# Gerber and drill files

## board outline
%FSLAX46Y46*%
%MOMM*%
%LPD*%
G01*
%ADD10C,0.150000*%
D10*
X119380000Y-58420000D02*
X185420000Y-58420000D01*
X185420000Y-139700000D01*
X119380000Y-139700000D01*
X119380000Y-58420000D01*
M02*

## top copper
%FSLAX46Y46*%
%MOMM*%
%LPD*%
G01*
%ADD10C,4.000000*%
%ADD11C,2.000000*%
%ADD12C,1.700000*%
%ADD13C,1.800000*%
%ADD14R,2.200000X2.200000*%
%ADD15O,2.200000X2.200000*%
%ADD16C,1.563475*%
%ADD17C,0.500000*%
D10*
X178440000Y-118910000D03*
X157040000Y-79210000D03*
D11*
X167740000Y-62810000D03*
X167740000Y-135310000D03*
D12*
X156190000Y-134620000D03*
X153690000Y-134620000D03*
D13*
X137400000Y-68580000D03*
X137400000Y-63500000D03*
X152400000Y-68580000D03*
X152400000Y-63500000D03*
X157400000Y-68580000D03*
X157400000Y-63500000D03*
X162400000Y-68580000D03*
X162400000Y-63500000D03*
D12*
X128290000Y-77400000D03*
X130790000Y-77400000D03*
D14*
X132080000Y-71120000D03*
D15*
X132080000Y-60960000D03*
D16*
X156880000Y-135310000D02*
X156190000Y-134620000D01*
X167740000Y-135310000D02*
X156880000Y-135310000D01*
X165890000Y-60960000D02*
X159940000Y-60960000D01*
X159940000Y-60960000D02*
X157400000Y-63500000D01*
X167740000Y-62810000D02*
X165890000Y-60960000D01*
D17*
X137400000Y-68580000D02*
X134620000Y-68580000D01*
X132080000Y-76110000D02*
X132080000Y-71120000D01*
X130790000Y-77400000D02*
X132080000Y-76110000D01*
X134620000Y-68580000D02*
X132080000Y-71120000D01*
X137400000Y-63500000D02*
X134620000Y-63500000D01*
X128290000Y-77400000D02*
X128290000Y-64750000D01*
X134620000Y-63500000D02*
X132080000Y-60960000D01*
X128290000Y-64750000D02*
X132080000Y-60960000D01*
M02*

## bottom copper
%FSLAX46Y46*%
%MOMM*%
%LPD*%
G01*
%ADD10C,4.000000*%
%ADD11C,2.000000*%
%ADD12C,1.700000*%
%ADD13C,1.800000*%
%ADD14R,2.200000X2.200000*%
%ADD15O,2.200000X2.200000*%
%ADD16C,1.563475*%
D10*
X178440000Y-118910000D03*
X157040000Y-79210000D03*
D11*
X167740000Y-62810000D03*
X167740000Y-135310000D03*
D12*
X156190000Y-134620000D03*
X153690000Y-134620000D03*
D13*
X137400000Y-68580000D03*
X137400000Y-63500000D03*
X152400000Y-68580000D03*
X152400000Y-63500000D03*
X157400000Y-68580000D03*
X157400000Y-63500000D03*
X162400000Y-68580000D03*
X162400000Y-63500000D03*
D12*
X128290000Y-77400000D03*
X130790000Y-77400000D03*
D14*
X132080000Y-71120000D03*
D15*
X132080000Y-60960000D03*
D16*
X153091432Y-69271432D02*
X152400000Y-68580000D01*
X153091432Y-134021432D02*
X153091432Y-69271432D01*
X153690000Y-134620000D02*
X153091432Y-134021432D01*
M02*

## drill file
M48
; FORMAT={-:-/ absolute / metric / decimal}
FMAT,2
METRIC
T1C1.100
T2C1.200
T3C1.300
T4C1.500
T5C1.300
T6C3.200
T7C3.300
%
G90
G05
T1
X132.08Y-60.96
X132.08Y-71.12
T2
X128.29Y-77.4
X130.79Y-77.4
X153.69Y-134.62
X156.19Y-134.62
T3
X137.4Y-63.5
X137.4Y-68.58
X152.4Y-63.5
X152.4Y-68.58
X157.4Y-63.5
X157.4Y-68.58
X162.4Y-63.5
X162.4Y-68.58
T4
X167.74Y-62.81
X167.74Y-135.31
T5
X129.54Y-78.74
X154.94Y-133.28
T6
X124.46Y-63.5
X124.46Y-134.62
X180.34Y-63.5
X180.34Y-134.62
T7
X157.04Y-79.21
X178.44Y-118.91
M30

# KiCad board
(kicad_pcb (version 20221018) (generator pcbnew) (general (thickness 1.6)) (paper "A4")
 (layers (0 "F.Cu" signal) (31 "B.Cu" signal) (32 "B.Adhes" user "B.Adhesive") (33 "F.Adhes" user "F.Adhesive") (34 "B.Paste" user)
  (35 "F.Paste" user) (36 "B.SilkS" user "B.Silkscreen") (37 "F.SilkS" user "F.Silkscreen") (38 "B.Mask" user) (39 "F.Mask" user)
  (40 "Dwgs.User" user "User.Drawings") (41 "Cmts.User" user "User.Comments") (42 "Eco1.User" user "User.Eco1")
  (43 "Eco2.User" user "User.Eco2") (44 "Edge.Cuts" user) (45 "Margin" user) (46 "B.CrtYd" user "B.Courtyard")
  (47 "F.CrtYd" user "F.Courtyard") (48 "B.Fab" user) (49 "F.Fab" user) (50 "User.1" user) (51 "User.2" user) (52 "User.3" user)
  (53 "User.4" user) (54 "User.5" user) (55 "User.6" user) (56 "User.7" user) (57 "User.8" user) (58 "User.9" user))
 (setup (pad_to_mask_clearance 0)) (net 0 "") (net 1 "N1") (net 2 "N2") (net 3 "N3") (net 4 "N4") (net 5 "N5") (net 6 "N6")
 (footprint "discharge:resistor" (layer "F.Cu") (at 152.74 124.56 90)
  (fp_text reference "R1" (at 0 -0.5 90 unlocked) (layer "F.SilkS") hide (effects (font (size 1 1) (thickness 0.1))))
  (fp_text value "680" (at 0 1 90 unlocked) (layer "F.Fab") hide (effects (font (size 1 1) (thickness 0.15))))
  (pad "" np_thru_hole circle (at 5.65 25.7 90) (size 4 4) (drill 3.3) (layers "F&B.Cu" "*.Mask"))
  (pad "" np_thru_hole circle (at 45.35 4.3 90) (size 4 4) (drill 3.3) (layers "F&B.Cu" "*.Mask"))
  (pad "1" thru_hole circle (at 61.75 15 90) (size 2 2) (drill 1.5) (layers "*.Cu" "*.Mask") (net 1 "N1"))
  (pad "2" thru_hole circle (at -10.75 15 90) (size 2 2) (drill 1.5) (layers "*.Cu" "*.Mask") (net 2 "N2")))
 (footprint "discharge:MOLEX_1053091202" (layer "F.Cu") (at 156.19 134.62 180)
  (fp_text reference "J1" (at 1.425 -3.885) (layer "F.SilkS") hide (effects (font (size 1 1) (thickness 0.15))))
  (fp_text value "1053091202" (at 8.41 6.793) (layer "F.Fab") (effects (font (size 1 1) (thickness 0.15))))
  (pad "" np_thru_hole circle (at 1.25 1.34 180) (size 1.3 1.3) (drill 1.3) (layers "*.Cu" "*.Mask"))
  (pad "1" thru_hole circle (at 0 0 180) (size 1.7 1.7) (drill 1.2) (layers "*.Cu") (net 2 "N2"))
  (pad "2" thru_hole circle (at 2.5 0 180) (size 1.7 1.7) (drill 1.2) (layers "*.Cu") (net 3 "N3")))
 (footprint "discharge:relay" (layer "F.Cu") (at 134.68 72.39 90)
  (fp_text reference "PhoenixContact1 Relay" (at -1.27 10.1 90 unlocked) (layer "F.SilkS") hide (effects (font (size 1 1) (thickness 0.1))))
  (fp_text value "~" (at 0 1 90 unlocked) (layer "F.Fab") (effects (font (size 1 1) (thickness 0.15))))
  (pad "1" thru_hole circle (at 3.81 2.72 90) (size 1.8 1.8) (drill 1.3) (layers "*.Cu" "*.Mask") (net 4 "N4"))
  (pad "2" thru_hole circle (at 8.89 2.72 90) (size 1.8 1.8) (drill 1.3) (layers "*.Cu" "*.Mask") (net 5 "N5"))
  (pad "3" thru_hole circle (at 3.81 17.72 90) (size 1.8 1.8) (drill 1.3) (layers "*.Cu" "*.Mask") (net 3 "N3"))
  (pad "3" thru_hole circle (at 8.89 17.72 90) (size 1.8 1.8) (drill 1.3) (layers "*.Cu" "*.Mask") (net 3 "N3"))
  (pad "4" thru_hole circle (at 3.81 22.72 90) (size 1.8 1.8) (drill 1.3) (layers "*.Cu" "*.Mask") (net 1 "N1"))
  (pad "4" thru_hole circle (at 8.89 22.72 90) (size 1.8 1.8) (drill 1.3) (layers "*.Cu" "*.Mask") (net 1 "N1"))
  (pad "5" thru_hole circle (at 3.81 27.72 90) (size 1.8 1.8) (drill 1.3) (layers "*.Cu" "*.Mask") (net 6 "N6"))
  (pad "5" thru_hole circle (at 8.89 27.72 90) (size 1.8 1.8) (drill 1.3) (layers "*.Cu" "*.Mask") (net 6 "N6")))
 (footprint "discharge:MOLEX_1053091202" (layer "F.Cu") (at 128.29 77.4)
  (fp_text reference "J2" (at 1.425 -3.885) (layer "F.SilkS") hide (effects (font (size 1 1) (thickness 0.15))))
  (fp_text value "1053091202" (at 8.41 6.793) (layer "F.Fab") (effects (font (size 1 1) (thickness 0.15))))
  (pad "" np_thru_hole circle (at 1.25 1.34) (size 1.3 1.3) (drill 1.3) (layers "*.Cu" "*.Mask"))
  (pad "1" thru_hole circle (at 0 0) (size 1.7 1.7) (drill 1.2) (layers "*.Cu") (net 5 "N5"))
  (pad "2" thru_hole circle (at 2.5 0) (size 1.7 1.7) (drill 1.2) (layers "*.Cu") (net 4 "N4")))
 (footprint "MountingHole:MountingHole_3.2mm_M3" (layer "F.Cu") (at 124.46 134.62)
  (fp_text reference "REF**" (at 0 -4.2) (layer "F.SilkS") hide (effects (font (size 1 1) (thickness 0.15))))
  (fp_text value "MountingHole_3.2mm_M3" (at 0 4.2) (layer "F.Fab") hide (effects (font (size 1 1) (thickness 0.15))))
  (pad "" np_thru_hole circle (at 0 0) (size 3.2 3.2) (drill 3.2) (layers "F&B.Cu" "*.Mask")))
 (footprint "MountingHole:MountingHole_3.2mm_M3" (layer "F.Cu") (at 124.46 63.5)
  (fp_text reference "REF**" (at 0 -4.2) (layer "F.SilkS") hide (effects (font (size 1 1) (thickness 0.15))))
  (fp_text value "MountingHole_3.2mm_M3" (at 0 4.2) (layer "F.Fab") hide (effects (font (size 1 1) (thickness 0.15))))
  (pad "" np_thru_hole circle (at 0 0) (size 3.2 3.2) (drill 3.2) (layers "F&B.Cu" "*.Mask")))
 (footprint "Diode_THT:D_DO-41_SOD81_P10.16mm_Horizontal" (layer "F.Cu") (at 132.08 71.12 90)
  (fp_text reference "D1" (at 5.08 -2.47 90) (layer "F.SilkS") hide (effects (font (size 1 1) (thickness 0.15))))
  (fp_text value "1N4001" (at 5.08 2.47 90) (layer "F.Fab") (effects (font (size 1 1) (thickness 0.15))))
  (pad "1" thru_hole rect (at 0 0 90) (size 2.2 2.2) (drill 1.1) (layers "*.Cu" "*.Mask") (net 4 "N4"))
  (pad "2" thru_hole oval (at 10.16 0 90) (size 2.2 2.2) (drill 1.1) (layers "*.Cu" "*.Mask") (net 5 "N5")))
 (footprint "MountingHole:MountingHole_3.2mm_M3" (layer "F.Cu") (at 180.34 63.5)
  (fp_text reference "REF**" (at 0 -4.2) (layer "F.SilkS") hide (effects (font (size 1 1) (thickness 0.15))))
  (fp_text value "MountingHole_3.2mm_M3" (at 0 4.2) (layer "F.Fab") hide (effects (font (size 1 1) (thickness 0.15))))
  (pad "" np_thru_hole circle (at 0 0) (size 3.2 3.2) (drill 3.2) (layers "*.Cu" "*.Mask")))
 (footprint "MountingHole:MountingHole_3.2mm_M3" (layer "F.Cu") (at 180.34 134.62)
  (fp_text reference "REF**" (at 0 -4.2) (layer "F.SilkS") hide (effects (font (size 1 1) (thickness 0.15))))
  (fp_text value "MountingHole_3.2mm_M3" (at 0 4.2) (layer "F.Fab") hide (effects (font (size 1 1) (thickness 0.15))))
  (pad "" np_thru_hole circle (at 0 0) (size 3.2 3.2) (drill 3.2) (layers "F&B.Cu" "*.Mask")))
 (gr_rect (start 119.38 58.42) (end 185.42 139.7) (stroke (width 0.15) (type default)) (fill none) (layer "Edge.Cuts"))
 (segment (start 153.091432 69.271432) (end 152.4 68.58) (width 1.563475) (layer "B.Cu") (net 3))
 (segment (start 153.091432 134.021432) (end 153.091432 69.271432) (width 1.563475) (layer "B.Cu") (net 3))
 (segment (start 153.69 134.62) (end 153.091432 134.021432) (width 1.563475) (layer "B.Cu") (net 3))
 (segment (start 156.88 135.31) (end 156.19 134.62) (width 1.563475) (layer "F.Cu") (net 2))
 (segment (start 167.74 135.31) (end 156.88 135.31) (width 1.563475) (layer "F.Cu") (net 2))
 (segment (start 165.89 60.96) (end 159.94 60.96) (width 1.563475) (layer "F.Cu") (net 1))
 (segment (start 159.94 60.96) (end 157.4 63.5) (width 1.563475) (layer "F.Cu") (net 1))
 (segment (start 167.74 62.81) (end 165.89 60.96) (width 1.563475) (layer "F.Cu") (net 1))
 (segment (start 137.4 68.58) (end 134.62 68.58) (width 0.5) (layer "F.Cu") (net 4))
 (segment (start 132.08 76.11) (end 132.08 71.12) (width 0.5) (layer "F.Cu") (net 4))
 (segment (start 130.79 77.4) (end 132.08 76.11) (width 0.5) (layer "F.Cu") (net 4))
 (segment (start 134.62 68.58) (end 132.08 71.12) (width 0.5) (layer "F.Cu") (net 4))
 (segment (start 137.4 63.5) (end 134.62 63.5) (width 0.5) (layer "F.Cu") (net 5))
 (segment (start 128.29 77.4) (end 128.29 64.75) (width 0.5) (layer "F.Cu") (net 5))
 (segment (start 134.62 63.5) (end 132.08 60.96) (width 0.5) (layer "F.Cu") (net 5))
 (segment (start 128.29 64.75) (end 132.08 60.96) (width 0.5) (layer "F.Cu") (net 5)))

